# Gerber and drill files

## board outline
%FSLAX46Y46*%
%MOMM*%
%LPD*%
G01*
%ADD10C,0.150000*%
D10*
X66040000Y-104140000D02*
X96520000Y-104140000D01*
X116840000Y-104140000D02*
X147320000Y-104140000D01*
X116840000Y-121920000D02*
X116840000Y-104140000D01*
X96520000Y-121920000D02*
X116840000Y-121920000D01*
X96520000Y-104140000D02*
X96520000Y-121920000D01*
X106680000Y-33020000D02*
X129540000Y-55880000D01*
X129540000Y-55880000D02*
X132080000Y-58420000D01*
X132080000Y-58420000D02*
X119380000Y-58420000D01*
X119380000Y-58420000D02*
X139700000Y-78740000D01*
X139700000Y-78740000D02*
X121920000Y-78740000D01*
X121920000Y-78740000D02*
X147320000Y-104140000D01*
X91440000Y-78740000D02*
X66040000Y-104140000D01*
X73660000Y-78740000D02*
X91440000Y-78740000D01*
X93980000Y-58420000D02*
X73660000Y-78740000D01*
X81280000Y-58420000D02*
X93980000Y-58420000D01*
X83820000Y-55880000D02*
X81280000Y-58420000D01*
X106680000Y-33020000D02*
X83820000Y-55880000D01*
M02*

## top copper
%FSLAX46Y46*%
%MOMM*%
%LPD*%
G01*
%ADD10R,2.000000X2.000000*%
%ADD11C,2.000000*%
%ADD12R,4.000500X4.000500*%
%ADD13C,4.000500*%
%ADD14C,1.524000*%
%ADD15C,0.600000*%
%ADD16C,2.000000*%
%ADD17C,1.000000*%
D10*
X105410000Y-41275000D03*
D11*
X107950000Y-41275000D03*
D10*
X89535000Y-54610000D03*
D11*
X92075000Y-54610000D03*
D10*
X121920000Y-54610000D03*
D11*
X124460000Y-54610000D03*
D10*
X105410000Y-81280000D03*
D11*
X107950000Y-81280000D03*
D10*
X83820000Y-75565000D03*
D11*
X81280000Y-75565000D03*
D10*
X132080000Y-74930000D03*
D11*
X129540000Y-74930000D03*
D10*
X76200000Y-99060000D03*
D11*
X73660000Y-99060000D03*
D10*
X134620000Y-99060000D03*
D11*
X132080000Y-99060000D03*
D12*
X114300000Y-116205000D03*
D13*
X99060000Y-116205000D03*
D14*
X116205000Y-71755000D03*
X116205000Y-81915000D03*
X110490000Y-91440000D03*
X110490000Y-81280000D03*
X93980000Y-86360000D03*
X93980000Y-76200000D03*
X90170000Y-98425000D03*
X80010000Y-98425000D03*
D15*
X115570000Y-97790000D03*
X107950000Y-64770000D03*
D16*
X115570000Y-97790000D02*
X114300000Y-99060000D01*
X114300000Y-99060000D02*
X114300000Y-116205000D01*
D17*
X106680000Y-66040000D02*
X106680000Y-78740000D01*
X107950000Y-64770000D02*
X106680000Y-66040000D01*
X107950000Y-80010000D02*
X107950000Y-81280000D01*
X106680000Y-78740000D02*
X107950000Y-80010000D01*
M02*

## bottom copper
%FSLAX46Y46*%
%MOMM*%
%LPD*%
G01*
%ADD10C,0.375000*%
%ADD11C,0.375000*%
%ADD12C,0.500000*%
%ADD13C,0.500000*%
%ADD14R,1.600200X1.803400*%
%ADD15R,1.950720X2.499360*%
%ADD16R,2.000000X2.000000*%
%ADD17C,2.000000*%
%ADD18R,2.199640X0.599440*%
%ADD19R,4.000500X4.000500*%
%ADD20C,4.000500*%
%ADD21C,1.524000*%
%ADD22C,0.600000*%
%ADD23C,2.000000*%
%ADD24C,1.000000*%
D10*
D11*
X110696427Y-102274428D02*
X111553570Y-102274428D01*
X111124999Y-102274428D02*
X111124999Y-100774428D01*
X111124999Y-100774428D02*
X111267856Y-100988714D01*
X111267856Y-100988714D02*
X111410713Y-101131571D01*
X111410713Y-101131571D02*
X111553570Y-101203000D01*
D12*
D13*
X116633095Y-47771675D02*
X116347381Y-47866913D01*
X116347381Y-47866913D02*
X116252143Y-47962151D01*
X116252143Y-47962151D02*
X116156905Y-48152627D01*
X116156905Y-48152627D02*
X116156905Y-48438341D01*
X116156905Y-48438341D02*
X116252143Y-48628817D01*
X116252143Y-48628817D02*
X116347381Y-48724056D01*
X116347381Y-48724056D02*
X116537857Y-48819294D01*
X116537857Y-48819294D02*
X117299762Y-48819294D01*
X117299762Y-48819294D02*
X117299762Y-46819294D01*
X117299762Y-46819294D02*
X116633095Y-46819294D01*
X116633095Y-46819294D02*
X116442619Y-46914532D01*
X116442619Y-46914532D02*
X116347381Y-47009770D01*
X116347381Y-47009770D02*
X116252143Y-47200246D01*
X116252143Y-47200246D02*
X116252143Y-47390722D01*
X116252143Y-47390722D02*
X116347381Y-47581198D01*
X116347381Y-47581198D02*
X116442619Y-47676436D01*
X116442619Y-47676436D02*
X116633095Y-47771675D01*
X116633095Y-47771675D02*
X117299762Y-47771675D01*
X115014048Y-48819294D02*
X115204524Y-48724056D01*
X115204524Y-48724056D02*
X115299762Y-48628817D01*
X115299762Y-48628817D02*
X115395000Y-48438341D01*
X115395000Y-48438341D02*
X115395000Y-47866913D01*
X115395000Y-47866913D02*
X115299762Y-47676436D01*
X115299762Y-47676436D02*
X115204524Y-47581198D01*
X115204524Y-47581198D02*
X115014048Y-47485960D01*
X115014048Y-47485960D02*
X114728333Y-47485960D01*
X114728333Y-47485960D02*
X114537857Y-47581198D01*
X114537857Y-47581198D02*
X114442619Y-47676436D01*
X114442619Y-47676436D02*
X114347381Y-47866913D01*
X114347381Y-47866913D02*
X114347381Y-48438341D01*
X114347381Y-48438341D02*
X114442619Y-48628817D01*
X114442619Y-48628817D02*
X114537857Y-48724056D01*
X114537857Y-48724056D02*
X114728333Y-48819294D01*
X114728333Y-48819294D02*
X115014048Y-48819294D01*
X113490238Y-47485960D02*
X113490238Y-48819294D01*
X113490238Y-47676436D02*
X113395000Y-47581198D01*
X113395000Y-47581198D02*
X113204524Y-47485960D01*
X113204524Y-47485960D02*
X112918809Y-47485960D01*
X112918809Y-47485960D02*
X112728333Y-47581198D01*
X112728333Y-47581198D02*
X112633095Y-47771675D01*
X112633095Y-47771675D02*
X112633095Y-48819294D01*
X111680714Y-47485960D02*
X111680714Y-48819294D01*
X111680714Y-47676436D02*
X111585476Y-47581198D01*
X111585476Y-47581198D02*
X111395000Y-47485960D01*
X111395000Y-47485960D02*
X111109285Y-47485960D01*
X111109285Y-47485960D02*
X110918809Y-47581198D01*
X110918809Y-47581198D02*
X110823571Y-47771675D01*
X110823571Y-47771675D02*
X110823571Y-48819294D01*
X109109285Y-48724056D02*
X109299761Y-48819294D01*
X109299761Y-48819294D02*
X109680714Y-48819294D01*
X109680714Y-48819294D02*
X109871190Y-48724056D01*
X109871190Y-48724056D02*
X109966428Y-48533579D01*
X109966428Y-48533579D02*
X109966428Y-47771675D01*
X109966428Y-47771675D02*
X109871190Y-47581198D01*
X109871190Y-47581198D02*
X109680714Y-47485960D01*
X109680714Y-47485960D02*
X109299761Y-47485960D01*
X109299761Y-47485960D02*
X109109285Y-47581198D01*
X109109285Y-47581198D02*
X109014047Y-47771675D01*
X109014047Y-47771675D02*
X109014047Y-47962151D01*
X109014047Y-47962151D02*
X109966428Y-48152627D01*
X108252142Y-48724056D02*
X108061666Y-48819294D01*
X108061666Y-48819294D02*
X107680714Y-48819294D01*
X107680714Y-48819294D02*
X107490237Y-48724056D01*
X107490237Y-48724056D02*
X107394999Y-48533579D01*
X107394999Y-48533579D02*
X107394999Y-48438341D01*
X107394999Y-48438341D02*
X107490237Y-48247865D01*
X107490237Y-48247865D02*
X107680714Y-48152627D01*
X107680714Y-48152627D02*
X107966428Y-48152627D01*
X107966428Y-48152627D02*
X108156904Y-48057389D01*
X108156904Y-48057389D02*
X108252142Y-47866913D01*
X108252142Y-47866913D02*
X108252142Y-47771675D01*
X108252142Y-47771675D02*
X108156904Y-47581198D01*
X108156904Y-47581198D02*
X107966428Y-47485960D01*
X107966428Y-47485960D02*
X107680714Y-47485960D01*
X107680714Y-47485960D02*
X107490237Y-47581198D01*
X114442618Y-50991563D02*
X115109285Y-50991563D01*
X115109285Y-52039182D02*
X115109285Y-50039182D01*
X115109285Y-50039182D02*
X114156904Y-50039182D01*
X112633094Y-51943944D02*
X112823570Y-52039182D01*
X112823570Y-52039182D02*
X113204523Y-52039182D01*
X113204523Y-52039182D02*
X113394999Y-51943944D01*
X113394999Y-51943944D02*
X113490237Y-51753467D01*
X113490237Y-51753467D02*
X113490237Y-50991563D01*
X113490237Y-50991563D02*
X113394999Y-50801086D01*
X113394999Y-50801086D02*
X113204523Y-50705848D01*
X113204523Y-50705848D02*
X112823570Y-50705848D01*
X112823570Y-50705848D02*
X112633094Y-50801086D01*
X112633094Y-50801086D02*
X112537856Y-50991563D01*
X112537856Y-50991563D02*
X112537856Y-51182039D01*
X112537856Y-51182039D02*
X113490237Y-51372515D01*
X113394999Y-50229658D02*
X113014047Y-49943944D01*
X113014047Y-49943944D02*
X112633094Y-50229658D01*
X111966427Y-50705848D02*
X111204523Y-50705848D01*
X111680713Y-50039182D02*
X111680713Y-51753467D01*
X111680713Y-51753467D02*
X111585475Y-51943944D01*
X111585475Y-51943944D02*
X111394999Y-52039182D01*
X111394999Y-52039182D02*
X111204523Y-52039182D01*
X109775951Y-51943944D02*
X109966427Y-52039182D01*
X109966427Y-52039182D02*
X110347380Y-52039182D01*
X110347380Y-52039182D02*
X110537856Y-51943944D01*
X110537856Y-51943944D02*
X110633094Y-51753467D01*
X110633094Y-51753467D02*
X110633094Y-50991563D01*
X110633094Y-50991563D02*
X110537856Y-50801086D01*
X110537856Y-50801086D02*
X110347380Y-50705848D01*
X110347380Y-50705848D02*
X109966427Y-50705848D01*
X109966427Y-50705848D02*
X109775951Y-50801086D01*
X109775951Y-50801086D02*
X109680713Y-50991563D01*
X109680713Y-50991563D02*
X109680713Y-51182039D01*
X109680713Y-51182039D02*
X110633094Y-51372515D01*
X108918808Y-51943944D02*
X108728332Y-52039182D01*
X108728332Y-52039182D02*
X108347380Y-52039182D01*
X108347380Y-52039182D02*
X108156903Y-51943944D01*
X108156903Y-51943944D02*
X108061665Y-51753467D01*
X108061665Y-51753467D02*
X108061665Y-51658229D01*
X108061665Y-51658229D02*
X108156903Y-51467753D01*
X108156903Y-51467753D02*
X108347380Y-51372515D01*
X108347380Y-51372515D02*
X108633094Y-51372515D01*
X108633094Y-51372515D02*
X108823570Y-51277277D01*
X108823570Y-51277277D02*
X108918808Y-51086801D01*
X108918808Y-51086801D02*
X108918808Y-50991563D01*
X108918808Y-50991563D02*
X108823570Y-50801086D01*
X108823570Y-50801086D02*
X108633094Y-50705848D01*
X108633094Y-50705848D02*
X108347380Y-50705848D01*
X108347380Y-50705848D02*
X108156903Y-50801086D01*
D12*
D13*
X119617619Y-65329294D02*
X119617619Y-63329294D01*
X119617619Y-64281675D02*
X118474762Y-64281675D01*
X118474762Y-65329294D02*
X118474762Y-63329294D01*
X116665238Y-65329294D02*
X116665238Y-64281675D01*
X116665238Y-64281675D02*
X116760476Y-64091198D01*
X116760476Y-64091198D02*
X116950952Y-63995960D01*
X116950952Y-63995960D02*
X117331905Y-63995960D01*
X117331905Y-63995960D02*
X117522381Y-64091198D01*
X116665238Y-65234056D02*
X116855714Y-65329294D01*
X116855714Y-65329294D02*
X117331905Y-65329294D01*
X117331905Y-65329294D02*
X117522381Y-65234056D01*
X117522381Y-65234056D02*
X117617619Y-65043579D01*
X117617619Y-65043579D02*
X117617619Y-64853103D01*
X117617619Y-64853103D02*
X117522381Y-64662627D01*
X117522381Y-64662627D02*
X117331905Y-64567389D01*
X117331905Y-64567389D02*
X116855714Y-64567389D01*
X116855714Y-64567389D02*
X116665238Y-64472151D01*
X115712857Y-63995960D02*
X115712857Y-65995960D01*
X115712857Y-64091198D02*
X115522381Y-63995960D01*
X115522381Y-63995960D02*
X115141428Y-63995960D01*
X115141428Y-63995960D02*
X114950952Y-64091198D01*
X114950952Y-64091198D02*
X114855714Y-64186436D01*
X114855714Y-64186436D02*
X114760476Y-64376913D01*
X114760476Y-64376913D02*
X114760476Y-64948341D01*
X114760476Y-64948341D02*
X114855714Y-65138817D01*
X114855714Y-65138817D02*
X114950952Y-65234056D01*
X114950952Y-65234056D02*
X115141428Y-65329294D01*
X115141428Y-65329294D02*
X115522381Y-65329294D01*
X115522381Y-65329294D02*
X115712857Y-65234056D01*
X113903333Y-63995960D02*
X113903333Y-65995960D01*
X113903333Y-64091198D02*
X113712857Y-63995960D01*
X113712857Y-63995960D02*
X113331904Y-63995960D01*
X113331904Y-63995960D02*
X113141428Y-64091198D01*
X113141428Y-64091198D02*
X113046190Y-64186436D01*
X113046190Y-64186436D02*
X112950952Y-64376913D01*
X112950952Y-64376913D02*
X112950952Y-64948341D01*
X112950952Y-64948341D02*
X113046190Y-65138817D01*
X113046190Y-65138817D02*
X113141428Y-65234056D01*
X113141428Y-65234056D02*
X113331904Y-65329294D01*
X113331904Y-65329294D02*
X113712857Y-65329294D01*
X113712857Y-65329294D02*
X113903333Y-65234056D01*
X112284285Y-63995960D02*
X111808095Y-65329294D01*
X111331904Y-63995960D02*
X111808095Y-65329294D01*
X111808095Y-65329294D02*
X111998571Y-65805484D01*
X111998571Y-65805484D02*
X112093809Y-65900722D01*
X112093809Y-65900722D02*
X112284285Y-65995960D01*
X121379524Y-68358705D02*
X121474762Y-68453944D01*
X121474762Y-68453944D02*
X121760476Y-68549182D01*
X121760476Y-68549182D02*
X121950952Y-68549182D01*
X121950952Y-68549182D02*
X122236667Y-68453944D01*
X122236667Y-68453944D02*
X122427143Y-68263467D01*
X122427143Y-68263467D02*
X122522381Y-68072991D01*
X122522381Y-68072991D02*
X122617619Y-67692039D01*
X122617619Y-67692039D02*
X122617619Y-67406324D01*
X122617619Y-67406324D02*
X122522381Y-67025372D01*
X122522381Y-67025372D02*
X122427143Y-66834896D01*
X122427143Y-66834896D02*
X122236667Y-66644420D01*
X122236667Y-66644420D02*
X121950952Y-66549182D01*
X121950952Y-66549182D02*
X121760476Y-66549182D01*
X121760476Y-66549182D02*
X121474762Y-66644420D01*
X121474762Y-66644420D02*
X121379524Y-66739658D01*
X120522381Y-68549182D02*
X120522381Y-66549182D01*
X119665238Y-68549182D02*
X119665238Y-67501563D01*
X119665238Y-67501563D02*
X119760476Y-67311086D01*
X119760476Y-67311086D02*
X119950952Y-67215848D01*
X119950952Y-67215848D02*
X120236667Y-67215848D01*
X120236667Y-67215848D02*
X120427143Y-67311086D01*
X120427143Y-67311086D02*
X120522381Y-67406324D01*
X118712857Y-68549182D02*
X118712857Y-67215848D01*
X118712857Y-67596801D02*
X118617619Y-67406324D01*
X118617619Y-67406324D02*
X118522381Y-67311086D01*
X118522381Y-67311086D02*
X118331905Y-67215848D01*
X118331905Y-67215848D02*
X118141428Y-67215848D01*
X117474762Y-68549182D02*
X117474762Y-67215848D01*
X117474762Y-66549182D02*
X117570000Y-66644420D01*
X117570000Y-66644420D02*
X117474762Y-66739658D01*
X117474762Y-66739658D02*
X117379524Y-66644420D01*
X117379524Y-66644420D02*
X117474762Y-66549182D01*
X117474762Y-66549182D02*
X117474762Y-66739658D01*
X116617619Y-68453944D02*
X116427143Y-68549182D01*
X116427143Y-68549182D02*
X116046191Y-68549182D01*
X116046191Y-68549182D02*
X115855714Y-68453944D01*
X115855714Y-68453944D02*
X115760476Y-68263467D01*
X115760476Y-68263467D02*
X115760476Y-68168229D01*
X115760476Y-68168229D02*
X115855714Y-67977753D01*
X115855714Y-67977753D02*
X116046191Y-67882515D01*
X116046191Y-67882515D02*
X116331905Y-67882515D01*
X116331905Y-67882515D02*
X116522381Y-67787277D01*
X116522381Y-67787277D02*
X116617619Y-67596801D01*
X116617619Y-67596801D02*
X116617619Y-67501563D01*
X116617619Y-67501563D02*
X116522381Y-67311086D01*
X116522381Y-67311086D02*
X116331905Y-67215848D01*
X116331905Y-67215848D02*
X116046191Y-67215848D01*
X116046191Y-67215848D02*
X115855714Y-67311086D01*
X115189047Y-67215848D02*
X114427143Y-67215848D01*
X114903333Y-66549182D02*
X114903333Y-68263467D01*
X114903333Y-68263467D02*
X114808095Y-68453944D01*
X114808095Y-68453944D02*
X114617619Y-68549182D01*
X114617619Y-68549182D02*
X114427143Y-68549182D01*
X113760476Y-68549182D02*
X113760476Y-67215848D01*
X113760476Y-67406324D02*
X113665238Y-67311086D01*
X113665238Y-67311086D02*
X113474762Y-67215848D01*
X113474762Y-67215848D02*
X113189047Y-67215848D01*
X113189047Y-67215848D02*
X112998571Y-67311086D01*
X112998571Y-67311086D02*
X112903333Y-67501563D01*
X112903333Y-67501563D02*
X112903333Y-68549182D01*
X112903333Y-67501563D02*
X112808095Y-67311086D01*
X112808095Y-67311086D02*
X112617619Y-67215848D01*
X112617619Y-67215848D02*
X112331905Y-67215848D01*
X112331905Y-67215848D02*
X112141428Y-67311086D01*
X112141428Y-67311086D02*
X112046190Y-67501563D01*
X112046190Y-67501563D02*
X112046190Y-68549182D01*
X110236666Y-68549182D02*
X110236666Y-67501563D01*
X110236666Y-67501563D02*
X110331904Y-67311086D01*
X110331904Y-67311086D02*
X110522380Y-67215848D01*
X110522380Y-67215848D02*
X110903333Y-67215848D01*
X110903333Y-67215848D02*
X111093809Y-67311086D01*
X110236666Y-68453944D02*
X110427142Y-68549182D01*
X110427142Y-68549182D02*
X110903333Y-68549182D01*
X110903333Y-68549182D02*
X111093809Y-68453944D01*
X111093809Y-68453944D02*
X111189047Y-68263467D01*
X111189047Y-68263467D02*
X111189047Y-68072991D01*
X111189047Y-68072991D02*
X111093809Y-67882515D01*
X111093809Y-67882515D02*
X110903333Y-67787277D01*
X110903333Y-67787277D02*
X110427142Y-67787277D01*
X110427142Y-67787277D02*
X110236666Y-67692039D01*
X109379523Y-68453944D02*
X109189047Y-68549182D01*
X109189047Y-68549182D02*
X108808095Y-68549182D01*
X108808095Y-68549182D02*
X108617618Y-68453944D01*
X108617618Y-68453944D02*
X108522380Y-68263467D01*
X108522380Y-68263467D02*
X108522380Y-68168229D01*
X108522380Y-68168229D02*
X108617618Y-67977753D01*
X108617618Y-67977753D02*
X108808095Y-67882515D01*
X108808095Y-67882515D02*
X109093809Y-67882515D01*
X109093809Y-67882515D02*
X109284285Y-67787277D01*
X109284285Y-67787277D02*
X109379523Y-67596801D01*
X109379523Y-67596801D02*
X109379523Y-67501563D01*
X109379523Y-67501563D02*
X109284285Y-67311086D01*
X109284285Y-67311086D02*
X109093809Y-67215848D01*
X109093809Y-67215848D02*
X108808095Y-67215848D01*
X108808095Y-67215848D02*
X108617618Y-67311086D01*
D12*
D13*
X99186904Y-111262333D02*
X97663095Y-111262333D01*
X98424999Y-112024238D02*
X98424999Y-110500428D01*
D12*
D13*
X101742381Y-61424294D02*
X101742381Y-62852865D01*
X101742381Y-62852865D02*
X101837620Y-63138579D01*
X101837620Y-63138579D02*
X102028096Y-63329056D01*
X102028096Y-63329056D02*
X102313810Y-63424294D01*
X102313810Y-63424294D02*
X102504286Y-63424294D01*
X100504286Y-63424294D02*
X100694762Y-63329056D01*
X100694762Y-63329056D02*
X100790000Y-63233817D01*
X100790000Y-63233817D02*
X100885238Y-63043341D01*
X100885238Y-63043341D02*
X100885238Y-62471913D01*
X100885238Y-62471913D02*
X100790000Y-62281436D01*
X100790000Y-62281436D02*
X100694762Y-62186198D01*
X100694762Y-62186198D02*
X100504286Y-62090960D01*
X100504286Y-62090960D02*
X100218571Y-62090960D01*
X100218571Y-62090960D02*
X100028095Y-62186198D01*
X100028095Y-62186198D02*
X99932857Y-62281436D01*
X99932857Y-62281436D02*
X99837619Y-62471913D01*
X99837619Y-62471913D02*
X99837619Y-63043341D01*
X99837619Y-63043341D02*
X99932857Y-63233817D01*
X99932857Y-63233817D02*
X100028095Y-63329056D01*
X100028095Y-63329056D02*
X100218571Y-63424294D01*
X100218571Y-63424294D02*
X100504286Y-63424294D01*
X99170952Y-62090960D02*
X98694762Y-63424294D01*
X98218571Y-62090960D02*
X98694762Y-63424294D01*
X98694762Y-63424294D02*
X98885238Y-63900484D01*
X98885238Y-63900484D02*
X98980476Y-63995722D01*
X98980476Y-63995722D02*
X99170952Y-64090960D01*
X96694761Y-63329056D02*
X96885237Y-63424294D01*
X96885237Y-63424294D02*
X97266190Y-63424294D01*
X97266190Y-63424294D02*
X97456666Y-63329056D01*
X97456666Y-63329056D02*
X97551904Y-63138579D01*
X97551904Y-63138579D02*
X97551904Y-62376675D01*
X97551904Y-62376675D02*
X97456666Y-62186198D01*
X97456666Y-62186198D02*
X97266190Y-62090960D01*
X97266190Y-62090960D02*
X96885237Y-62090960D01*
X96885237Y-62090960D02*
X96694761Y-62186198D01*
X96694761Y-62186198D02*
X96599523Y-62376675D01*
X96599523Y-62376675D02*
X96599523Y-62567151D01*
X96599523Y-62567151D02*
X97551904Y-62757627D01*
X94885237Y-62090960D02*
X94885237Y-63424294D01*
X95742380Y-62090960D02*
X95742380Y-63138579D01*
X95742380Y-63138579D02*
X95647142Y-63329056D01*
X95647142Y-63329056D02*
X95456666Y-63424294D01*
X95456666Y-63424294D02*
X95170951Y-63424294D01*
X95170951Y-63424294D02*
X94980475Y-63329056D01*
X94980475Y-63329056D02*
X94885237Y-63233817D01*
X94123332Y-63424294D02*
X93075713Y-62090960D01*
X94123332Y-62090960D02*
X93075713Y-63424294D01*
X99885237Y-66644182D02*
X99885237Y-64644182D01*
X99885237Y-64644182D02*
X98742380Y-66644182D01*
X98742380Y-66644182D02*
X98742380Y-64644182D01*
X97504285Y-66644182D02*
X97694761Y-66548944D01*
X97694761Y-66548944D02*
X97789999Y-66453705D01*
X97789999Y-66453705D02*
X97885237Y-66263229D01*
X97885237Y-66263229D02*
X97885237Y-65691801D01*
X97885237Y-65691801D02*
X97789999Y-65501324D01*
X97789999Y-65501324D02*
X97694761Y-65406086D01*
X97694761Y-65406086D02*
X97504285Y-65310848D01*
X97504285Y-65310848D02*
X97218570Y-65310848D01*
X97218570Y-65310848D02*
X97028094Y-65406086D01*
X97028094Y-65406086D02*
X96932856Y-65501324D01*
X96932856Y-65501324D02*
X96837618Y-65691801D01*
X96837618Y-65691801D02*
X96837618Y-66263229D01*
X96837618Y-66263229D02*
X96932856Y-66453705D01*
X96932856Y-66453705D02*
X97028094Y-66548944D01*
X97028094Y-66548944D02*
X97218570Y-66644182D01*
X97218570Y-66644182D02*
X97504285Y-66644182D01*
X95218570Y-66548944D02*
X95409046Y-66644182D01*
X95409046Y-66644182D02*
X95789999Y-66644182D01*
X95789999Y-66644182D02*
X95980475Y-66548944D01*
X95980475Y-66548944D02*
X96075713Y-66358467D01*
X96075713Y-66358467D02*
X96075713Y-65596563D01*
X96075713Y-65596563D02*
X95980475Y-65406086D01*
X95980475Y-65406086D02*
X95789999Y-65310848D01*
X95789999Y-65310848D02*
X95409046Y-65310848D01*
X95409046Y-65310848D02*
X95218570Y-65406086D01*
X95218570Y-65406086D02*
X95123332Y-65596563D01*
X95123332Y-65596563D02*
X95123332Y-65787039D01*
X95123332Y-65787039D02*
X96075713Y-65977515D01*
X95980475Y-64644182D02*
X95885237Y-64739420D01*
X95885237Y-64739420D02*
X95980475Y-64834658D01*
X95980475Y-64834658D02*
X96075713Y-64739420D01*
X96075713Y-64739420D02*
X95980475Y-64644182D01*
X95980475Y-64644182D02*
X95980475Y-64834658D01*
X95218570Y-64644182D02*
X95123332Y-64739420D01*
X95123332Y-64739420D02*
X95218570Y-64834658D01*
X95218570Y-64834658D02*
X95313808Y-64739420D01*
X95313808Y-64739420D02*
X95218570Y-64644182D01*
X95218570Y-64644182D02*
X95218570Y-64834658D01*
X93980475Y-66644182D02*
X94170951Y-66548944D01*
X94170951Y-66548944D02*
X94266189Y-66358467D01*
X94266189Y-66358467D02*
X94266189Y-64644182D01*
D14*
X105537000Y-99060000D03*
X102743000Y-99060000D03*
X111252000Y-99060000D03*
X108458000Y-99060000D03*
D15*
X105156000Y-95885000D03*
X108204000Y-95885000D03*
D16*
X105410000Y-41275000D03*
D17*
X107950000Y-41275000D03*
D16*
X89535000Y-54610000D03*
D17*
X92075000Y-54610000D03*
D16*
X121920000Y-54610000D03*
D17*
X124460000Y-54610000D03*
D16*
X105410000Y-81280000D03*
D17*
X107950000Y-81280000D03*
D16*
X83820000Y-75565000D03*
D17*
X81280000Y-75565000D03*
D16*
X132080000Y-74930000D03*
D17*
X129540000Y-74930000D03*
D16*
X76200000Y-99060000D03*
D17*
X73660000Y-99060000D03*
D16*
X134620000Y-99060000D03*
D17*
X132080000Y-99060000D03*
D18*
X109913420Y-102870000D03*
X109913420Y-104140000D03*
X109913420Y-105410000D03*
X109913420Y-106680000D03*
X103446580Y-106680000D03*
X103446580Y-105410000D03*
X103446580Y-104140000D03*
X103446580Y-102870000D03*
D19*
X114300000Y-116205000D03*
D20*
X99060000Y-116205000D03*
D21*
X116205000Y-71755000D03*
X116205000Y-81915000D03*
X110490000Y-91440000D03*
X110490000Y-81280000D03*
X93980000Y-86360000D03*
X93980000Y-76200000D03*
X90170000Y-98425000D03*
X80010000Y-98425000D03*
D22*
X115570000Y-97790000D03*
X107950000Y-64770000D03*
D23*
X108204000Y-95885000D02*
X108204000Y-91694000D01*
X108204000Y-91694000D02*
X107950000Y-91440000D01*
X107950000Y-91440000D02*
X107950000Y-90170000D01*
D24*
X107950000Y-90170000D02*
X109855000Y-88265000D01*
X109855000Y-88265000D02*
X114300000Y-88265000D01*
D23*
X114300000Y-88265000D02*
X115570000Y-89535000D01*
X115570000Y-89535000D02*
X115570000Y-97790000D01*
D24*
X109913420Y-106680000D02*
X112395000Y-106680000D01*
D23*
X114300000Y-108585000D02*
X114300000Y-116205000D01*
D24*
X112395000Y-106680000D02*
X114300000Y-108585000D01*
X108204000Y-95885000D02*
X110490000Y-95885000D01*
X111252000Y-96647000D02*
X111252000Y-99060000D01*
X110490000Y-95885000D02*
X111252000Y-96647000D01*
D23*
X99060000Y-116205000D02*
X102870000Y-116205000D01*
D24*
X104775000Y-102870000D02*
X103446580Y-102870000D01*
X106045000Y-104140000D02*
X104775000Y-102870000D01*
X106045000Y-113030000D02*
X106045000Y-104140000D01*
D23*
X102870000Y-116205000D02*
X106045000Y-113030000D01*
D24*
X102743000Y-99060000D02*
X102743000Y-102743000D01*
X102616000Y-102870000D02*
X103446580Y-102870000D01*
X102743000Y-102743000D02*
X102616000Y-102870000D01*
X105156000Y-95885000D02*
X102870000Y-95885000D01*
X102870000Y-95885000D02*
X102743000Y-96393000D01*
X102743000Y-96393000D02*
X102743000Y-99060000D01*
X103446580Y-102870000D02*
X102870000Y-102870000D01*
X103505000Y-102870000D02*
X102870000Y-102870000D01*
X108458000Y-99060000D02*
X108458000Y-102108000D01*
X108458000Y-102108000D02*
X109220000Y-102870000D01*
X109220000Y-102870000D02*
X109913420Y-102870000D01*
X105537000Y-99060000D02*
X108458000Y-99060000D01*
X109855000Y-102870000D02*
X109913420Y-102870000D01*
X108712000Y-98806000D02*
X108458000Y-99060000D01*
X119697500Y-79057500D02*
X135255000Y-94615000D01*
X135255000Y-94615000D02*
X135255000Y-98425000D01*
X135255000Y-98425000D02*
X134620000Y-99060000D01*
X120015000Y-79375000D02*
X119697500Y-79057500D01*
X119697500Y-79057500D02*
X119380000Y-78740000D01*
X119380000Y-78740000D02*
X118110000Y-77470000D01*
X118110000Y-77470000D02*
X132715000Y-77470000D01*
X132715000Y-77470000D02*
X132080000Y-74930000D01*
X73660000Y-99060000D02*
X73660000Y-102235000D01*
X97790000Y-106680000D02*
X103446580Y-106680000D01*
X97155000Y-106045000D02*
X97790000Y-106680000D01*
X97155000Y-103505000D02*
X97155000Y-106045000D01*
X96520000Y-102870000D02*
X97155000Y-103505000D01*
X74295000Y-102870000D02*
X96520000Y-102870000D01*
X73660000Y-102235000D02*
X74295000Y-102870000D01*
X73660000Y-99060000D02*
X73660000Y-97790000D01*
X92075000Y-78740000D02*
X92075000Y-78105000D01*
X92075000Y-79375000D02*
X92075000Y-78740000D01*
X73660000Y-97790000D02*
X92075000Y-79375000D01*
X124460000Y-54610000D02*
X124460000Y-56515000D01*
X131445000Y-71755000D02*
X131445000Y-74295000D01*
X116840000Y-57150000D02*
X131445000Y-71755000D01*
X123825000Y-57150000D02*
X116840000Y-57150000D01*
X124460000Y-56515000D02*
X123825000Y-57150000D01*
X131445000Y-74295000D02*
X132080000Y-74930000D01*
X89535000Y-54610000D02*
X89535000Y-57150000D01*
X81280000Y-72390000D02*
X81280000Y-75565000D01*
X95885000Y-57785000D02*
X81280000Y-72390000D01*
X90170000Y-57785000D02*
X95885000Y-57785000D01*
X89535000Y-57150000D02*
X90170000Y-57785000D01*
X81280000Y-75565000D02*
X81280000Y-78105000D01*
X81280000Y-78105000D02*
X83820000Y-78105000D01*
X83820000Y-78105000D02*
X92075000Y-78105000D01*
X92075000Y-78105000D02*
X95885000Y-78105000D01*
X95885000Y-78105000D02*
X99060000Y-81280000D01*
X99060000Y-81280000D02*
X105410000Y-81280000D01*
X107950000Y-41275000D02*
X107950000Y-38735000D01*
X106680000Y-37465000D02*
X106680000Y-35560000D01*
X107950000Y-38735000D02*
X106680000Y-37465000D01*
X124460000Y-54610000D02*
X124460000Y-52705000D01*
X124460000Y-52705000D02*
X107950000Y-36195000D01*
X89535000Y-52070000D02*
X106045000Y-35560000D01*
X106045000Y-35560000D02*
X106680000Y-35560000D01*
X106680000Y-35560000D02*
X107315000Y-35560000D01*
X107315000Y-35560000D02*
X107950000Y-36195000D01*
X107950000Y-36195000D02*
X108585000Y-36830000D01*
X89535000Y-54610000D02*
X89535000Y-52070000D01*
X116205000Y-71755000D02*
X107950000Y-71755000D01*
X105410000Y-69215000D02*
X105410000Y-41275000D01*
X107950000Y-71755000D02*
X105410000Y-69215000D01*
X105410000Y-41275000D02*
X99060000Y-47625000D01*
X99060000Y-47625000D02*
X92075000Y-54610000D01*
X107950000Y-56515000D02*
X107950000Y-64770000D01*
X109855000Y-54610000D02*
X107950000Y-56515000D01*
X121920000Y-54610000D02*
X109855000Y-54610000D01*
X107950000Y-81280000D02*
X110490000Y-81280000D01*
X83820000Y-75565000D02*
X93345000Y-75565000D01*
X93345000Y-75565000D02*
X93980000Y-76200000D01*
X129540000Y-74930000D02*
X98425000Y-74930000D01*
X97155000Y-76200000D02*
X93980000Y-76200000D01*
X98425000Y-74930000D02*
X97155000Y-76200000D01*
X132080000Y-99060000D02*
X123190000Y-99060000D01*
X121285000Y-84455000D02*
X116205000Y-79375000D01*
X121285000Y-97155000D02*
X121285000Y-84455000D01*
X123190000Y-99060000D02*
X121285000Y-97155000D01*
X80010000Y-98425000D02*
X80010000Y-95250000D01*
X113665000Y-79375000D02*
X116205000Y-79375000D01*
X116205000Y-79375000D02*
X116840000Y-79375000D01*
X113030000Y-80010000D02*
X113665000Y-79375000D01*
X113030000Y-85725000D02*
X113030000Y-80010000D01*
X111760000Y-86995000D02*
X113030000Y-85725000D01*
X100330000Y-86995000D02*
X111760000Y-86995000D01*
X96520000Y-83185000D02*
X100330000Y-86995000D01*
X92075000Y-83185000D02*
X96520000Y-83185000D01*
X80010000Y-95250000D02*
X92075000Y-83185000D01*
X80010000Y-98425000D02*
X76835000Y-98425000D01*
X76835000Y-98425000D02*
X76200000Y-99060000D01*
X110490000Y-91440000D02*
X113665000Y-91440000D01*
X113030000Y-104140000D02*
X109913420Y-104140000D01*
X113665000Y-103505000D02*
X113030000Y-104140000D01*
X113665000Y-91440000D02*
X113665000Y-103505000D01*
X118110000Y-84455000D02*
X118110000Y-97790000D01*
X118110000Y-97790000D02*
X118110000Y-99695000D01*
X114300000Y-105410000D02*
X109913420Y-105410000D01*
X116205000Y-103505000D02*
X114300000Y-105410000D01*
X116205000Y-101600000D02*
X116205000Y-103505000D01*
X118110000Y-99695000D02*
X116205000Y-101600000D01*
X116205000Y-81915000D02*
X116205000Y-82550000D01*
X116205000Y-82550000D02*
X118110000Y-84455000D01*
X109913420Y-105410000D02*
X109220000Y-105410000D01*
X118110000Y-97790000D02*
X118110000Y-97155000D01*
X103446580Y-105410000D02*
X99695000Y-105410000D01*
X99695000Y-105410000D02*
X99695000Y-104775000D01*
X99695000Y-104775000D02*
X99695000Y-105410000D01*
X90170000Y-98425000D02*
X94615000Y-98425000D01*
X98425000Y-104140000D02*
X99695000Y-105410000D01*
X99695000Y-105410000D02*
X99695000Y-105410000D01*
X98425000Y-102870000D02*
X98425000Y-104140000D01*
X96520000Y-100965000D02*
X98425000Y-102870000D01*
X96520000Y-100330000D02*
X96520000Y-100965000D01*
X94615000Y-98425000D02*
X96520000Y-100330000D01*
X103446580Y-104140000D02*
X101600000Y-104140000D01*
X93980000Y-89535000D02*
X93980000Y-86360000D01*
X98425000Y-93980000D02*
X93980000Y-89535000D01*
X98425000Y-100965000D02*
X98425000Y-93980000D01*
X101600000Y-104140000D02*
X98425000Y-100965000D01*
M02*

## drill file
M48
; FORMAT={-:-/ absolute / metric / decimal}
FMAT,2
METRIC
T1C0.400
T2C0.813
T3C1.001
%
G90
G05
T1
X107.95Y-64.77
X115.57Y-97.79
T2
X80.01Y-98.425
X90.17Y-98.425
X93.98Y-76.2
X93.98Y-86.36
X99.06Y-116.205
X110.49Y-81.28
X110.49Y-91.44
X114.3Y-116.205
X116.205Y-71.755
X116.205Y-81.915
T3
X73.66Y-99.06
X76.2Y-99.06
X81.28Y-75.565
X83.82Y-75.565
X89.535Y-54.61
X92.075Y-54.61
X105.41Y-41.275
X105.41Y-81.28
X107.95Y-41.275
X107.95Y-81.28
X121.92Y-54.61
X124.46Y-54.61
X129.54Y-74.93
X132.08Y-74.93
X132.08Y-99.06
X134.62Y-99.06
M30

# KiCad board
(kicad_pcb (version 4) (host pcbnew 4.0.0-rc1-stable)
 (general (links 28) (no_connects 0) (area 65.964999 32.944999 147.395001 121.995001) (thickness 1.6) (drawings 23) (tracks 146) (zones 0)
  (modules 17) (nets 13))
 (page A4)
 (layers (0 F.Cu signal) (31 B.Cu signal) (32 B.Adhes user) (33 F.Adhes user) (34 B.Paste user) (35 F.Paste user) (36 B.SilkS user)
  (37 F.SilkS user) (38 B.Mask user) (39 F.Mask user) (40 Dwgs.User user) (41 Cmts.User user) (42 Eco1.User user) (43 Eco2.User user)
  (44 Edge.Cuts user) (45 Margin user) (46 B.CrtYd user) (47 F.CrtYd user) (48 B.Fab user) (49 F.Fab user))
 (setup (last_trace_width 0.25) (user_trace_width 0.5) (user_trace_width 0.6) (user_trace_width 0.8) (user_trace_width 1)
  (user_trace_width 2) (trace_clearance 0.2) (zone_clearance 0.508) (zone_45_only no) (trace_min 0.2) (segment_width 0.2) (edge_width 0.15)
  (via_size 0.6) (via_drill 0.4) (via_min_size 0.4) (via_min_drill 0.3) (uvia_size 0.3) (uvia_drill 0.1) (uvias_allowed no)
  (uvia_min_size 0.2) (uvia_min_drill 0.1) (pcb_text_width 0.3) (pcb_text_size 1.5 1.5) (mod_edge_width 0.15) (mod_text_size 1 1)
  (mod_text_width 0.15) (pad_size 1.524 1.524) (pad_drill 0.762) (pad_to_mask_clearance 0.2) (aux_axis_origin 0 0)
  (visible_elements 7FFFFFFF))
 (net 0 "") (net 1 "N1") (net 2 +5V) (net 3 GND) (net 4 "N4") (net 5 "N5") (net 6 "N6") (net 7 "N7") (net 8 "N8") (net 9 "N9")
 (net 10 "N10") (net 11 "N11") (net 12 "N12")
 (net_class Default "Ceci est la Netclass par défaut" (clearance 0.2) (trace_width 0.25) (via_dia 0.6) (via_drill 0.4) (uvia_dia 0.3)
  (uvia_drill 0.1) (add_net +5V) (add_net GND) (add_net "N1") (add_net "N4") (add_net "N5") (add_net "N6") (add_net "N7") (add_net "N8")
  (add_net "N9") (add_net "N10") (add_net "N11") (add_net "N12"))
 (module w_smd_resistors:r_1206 (layer B.Cu) (at 104.14 99.06)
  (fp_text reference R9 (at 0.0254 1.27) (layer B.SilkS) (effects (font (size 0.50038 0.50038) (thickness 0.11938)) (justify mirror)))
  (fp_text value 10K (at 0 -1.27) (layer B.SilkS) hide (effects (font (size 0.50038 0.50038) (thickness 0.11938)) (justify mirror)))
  (pad 1 smd rect (at 1.397 0) (size 1.6002 1.8034) (layers B.Cu B.Paste B.Mask) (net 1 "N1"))
  (pad 2 smd rect (at -1.397 0) (size 1.6002 1.8034) (layers B.Cu B.Paste B.Mask) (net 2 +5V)))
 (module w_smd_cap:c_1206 (layer B.Cu) (at 109.855 99.06)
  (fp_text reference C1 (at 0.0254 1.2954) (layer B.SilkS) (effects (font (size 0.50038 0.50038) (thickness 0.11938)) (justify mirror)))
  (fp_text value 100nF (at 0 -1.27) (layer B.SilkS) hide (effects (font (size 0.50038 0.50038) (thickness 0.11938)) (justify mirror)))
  (pad 1 smd rect (at 1.397 0) (size 1.6002 1.8034) (layers B.Cu B.Paste B.Mask) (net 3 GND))
  (pad 2 smd rect (at -1.397 0) (size 1.6002 1.8034) (layers B.Cu B.Paste B.Mask) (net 1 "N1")))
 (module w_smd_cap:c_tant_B (layer B.Cu) (at 106.68 95.885 180)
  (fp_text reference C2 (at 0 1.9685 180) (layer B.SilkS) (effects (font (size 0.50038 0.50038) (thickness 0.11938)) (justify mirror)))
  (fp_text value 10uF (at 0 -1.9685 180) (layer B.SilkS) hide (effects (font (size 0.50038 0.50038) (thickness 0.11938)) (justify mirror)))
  (pad 1 smd rect (at 1.524 0 180) (size 1.95072 2.49936) (layers B.Cu B.Paste B.Mask) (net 2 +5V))
  (pad 2 smd rect (at -1.524 0 180) (size 1.95072 2.49936) (layers B.Cu B.Paste B.Mask) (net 3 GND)))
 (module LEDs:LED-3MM (layer F.Cu) (at 105.41 41.275)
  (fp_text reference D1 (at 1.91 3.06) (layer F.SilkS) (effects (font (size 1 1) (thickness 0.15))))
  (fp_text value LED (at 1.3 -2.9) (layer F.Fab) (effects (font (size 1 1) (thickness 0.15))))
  (pad 1 thru_hole rect (at 0 0 90) (size 2 2) (drill 1.00076) (layers *.Cu *.Mask F.SilkS) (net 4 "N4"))
  (pad 2 thru_hole circle (at 2.54 0) (size 2 2) (drill 1.00076) (layers *.Cu *.Mask F.SilkS) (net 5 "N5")))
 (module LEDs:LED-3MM (layer F.Cu) (at 89.535 54.61)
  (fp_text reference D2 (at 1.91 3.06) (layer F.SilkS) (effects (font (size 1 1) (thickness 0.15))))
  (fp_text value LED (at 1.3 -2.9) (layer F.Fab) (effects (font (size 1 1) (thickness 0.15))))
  (pad 1 thru_hole rect (at 0 0 90) (size 2 2) (drill 1.00076) (layers *.Cu *.Mask F.SilkS) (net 5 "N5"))
  (pad 2 thru_hole circle (at 2.54 0) (size 2 2) (drill 1.00076) (layers *.Cu *.Mask F.SilkS) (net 4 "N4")))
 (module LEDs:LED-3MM (layer F.Cu) (at 121.92 54.61)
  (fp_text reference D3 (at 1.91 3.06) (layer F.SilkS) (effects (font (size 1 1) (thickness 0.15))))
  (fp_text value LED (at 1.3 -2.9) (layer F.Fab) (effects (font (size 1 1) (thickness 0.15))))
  (pad 1 thru_hole rect (at 0 0 90) (size 2 2) (drill 1.00076) (layers *.Cu *.Mask F.SilkS) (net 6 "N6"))
  (pad 2 thru_hole circle (at 2.54 0) (size 2 2) (drill 1.00076) (layers *.Cu *.Mask F.SilkS) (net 5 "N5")))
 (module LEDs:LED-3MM (layer F.Cu) (at 105.41 81.28)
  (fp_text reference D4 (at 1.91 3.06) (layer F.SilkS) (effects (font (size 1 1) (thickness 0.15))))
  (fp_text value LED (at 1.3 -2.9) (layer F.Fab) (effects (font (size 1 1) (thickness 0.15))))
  (pad 1 thru_hole rect (at 0 0 90) (size 2 2) (drill 1.00076) (layers *.Cu *.Mask F.SilkS) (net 5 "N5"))
  (pad 2 thru_hole circle (at 2.54 0) (size 2 2) (drill 1.00076) (layers *.Cu *.Mask F.SilkS) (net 6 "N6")))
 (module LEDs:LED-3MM (layer F.Cu) (at 83.82 75.565 180)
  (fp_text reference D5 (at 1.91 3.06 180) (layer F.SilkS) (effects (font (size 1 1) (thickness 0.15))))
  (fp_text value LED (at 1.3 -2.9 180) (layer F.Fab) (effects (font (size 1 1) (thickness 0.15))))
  (pad 1 thru_hole rect (at 0 0 270) (size 2 2) (drill 1.00076) (layers *.Cu *.Mask F.SilkS) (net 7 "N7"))
  (pad 2 thru_hole circle (at 2.54 0 180) (size 2 2) (drill 1.00076) (layers *.Cu *.Mask F.SilkS) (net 5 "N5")))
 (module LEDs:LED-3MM (layer F.Cu) (at 132.08 74.93 180)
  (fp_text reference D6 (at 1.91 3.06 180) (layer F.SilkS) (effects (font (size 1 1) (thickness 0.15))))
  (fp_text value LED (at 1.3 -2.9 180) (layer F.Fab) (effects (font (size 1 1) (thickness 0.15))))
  (pad 1 thru_hole rect (at 0 0 270) (size 2 2) (drill 1.00076) (layers *.Cu *.Mask F.SilkS) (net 5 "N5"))
  (pad 2 thru_hole circle (at 2.54 0 180) (size 2 2) (drill 1.00076) (layers *.Cu *.Mask F.SilkS) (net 7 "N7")))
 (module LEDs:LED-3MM (layer F.Cu) (at 76.2 99.06 180)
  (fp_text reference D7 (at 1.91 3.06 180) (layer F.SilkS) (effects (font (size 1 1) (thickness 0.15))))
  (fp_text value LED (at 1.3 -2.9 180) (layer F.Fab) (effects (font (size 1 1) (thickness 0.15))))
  (pad 1 thru_hole rect (at 0 0 270) (size 2 2) (drill 1.00076) (layers *.Cu *.Mask F.SilkS) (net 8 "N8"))
  (pad 2 thru_hole circle (at 2.54 0 180) (size 2 2) (drill 1.00076) (layers *.Cu *.Mask F.SilkS) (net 5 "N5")))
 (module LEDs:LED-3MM (layer F.Cu) (at 134.62 99.06 180)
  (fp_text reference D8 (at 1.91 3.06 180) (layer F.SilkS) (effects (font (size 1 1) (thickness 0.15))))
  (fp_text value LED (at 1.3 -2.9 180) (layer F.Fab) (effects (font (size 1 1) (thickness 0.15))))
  (pad 1 thru_hole rect (at 0 0 270) (size 2 2) (drill 1.00076) (layers *.Cu *.Mask F.SilkS) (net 5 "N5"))
  (pad 2 thru_hole circle (at 2.54 0 180) (size 2 2) (drill 1.00076) (layers *.Cu *.Mask F.SilkS) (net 8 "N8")))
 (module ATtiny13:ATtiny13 (layer B.Cu) (at 106.045 104.775 270)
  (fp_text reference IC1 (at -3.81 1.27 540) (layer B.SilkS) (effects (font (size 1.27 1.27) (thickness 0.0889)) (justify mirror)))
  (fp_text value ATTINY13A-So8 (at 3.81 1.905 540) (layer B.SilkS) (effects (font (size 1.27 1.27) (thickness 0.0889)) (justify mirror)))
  (pad 1 smd rect (at -1.905 -3.86842 270) (size 0.59944 2.19964) (layers B.Cu B.Paste B.Mask) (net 1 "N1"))
  (pad 2 smd rect (at -0.635 -3.86842 270) (size 0.59944 2.19964) (layers B.Cu B.Paste B.Mask) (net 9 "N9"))
  (pad 3 smd rect (at 0.635 -3.86842 270) (size 0.59944 2.19964) (layers B.Cu B.Paste B.Mask) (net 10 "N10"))
  (pad 4 smd rect (at 1.905 -3.86842 270) (size 0.59944 2.19964) (layers B.Cu B.Paste B.Mask) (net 3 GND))
  (pad 5 smd rect (at 1.905 2.59842 270) (size 0.59944 2.19964) (layers B.Cu B.Paste B.Mask) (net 5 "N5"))
  (pad 6 smd rect (at 0.635 2.59842 270) (size 0.59944 2.19964) (layers B.Cu B.Paste B.Mask) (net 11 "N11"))
  (pad 7 smd rect (at -0.635 2.59842 270) (size 0.59944 2.19964) (layers B.Cu B.Paste B.Mask) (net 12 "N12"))
  (pad 8 smd rect (at -1.905 2.59842 270) (size 0.59944 2.19964) (layers B.Cu B.Paste B.Mask) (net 2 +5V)))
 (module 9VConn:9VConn (layer F.Cu) (at 106.68 116.205)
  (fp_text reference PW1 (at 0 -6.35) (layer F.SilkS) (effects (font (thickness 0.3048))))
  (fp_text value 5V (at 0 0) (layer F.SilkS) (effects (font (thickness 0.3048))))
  (pad 1 thru_hole rect (at 7.62 0) (size 4.0005 4.0005) (drill 0.8128) (layers *.Cu *.Mask F.SilkS) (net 3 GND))
  (pad 2 thru_hole circle (at -7.62 0) (size 4.0005 4.0005) (drill 0.8128) (layers *.Cu *.Mask F.SilkS) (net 2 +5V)))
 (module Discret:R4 (layer B.Cu) (at 116.205 76.835 270)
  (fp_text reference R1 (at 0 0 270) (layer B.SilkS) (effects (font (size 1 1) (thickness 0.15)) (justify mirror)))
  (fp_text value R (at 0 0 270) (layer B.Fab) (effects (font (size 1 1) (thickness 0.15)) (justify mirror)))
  (pad 1 thru_hole circle (at -5.08 0 270) (size 1.524 1.524) (drill 0.8128) (layers *.Cu *.Mask B.SilkS) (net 4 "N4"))
  (pad 2 thru_hole circle (at 5.08 0 270) (size 1.524 1.524) (drill 0.8128) (layers *.Cu *.Mask B.SilkS) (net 10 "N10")))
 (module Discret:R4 (layer B.Cu) (at 110.49 86.36 90)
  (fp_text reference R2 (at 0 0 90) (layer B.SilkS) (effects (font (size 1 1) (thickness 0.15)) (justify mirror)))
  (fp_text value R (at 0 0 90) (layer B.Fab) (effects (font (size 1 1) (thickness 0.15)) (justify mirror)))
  (pad 1 thru_hole circle (at -5.08 0 90) (size 1.524 1.524) (drill 0.8128) (layers *.Cu *.Mask B.SilkS) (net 9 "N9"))
  (pad 2 thru_hole circle (at 5.08 0 90) (size 1.524 1.524) (drill 0.8128) (layers *.Cu *.Mask B.SilkS) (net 6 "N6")))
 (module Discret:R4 (layer B.Cu) (at 93.98 81.28 90)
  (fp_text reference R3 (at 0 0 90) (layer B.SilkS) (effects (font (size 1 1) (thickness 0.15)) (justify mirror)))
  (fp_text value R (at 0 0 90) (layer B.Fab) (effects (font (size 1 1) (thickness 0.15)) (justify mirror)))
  (pad 1 thru_hole circle (at -5.08 0 90) (size 1.524 1.524) (drill 0.8128) (layers *.Cu *.Mask B.SilkS) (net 12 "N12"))
  (pad 2 thru_hole circle (at 5.08 0 90) (size 1.524 1.524) (drill 0.8128) (layers *.Cu *.Mask B.SilkS) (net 7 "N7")))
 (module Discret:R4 (layer B.Cu) (at 85.09 98.425 180)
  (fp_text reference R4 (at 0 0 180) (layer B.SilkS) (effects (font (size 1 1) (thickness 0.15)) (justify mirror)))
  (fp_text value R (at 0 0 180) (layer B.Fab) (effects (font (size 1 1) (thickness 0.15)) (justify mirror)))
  (pad 1 thru_hole circle (at -5.08 0 180) (size 1.524 1.524) (drill 0.8128) (layers *.Cu *.Mask B.SilkS) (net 11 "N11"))
  (pad 2 thru_hole circle (at 5.08 0 180) (size 1.524 1.524) (drill 0.8128) (layers *.Cu *.Mask B.SilkS) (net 8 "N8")))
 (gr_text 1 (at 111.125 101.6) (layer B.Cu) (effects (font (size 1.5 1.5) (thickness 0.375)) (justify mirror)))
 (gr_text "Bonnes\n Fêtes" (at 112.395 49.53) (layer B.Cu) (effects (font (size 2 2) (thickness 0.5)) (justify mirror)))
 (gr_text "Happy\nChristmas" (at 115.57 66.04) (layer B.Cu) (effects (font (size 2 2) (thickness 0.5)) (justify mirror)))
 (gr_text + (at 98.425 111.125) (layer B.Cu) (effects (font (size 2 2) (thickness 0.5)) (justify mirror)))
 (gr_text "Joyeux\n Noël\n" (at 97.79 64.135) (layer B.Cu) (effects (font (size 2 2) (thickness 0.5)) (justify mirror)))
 (gr_line (start 66.04 104.14) (end 96.52 104.14) (angle 90) (layer Edge.Cuts) (width 0.15))
 (gr_line (start 116.84 104.14) (end 147.32 104.14) (angle 90) (layer Edge.Cuts) (width 0.15))
 (gr_line (start 116.84 121.92) (end 116.84 104.14) (angle 90) (layer Edge.Cuts) (width 0.15))
 (gr_line (start 96.52 121.92) (end 116.84 121.92) (angle 90) (layer Edge.Cuts) (width 0.15))
 (gr_line (start 96.52 104.14) (end 96.52 121.92) (angle 90) (layer Edge.Cuts) (width 0.15))
 (gr_line (start 106.68 33.02) (end 129.54 55.88) (angle 90) (layer Edge.Cuts) (width 0.15))
 (gr_line (start 129.54 55.88) (end 132.08 58.42) (angle 90) (layer Edge.Cuts) (width 0.15))
 (gr_line (start 132.08 58.42) (end 119.38 58.42) (angle 90) (layer Edge.Cuts) (width 0.15))
 (gr_line (start 119.38 58.42) (end 139.7 78.74) (angle 90) (layer Edge.Cuts) (width 0.15))
 (gr_line (start 139.7 78.74) (end 121.92 78.74) (angle 90) (layer Edge.Cuts) (width 0.15))
 (gr_line (start 121.92 78.74) (end 147.32 104.14) (angle 90) (layer Edge.Cuts) (width 0.15))
 (gr_line (start 91.44 78.74) (end 66.04 104.14) (angle 90) (layer Edge.Cuts) (width 0.15))
 (gr_line (start 73.66 78.74) (end 91.44 78.74) (angle 90) (layer Edge.Cuts) (width 0.15))
 (gr_line (start 93.98 58.42) (end 73.66 78.74) (angle 90) (layer Edge.Cuts) (width 0.15))
 (gr_line (start 81.28 58.42) (end 93.98 58.42) (angle 90) (layer Edge.Cuts) (width 0.15))
 (gr_line (start 83.82 55.88) (end 81.28 58.42) (angle 90) (layer Edge.Cuts) (width 0.15))
 (gr_line (start 106.68 33.02) (end 83.82 55.88) (angle 90) (layer Edge.Cuts) (width 0.15))
 (segment (start 108.204 95.885) (end 108.204 91.694) (width 2) (layer B.Cu) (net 3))
 (segment (start 108.204 91.694) (end 107.95 91.44) (width 2) (layer B.Cu) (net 3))
 (segment (start 107.95 91.44) (end 107.95 90.17) (width 2) (layer B.Cu) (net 3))
 (segment (start 107.95 90.17) (end 109.855 88.265) (width 1) (layer B.Cu) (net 3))
 (segment (start 109.855 88.265) (end 114.3 88.265) (width 1) (layer B.Cu) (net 3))
 (segment (start 114.3 88.265) (end 115.57 89.535) (width 2) (layer B.Cu) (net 3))
 (segment (start 115.57 89.535) (end 115.57 97.79) (width 2) (layer B.Cu) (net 3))
 (via (at 115.57 97.79) (size 0.6) (drill 0.4) (layers F.Cu B.Cu) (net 3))
 (segment (start 115.57 97.79) (end 114.3 99.06) (width 2) (layer F.Cu) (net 3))
 (segment (start 114.3 99.06) (end 114.3 116.205) (width 2) (layer F.Cu) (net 3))
 (segment (start 109.91342 106.68) (end 112.395 106.68) (width 1) (layer B.Cu) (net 3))
 (segment (start 114.3 108.585) (end 114.3 116.205) (width 2) (layer B.Cu) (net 3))
 (segment (start 112.395 106.68) (end 114.3 108.585) (width 1) (layer B.Cu) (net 3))
 (segment (start 108.204 95.885) (end 110.49 95.885) (width 1) (layer B.Cu) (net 3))
 (segment (start 111.252 96.647) (end 111.252 99.06) (width 1) (layer B.Cu) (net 3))
 (segment (start 110.49 95.885) (end 111.252 96.647) (width 1) (layer B.Cu) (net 3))
 (segment (start 99.06 116.205) (end 102.87 116.205) (width 2) (layer B.Cu) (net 2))
 (segment (start 104.775 102.87) (end 103.44658 102.87) (width 1) (layer B.Cu) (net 2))
 (segment (start 106.045 104.14) (end 104.775 102.87) (width 1) (layer B.Cu) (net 2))
 (segment (start 106.045 113.03) (end 106.045 104.14) (width 1) (layer B.Cu) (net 2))
 (segment (start 102.87 116.205) (end 106.045 113.03) (width 2) (layer B.Cu) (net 2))
 (segment (start 102.743 99.06) (end 102.743 102.743) (width 1) (layer B.Cu) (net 2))
 (segment (start 102.616 102.87) (end 103.44658 102.87) (width 1) (layer B.Cu) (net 2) (status 20))
 (segment (start 102.743 102.743) (end 102.616 102.87) (width 1) (layer B.Cu) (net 2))
 (segment (start 105.156 95.885) (end 102.87 95.885) (width 1) (layer B.Cu) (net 2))
 (segment (start 102.87 95.885) (end 102.743 96.393) (width 1) (layer B.Cu) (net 2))
 (segment (start 102.743 96.393) (end 102.743 99.06) (width 1) (layer B.Cu) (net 2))
 (segment (start 103.44658 102.87) (end 102.87 102.87) (width 1) (layer B.Cu) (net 2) (status 10))
 (segment (start 103.505 102.87) (end 102.87 102.87) (width 1) (layer B.Cu) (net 2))
 (segment (start 108.458 99.06) (end 108.458 102.108) (width 1) (layer B.Cu) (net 1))
 (segment (start 108.458 102.108) (end 109.22 102.87) (width 1) (layer B.Cu) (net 1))
 (segment (start 109.22 102.87) (end 109.91342 102.87) (width 1) (layer B.Cu) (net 1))
 (segment (start 105.537 99.06) (end 108.458 99.06) (width 1) (layer B.Cu) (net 1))
 (segment (start 109.855 102.87) (end 109.91342 102.87) (width 1) (layer B.Cu) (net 1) (status 30))
 (segment (start 108.712 98.806) (end 108.458 99.06) (width 1) (layer B.Cu) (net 1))
 (segment (start 119.6975 79.0575) (end 135.255 94.615) (width 1) (layer B.Cu) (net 5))
 (segment (start 135.255 94.615) (end 135.255 98.425) (width 1) (layer B.Cu) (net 5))
 (segment (start 135.255 98.425) (end 134.62 99.06) (width 1) (layer B.Cu) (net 5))
 (segment (start 120.015 79.375) (end 119.6975 79.0575) (width 1) (layer B.Cu) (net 5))
 (segment (start 119.6975 79.0575) (end 119.38 78.74) (width 1) (layer B.Cu) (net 5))
 (segment (start 119.38 78.74) (end 118.11 77.47) (width 1) (layer B.Cu) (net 5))
 (segment (start 118.11 77.47) (end 132.715 77.47) (width 1) (layer B.Cu) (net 5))
 (segment (start 132.715 77.47) (end 132.08 74.93) (width 1) (layer B.Cu) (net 5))
 (segment (start 73.66 99.06) (end 73.66 102.235) (width 1) (layer B.Cu) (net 5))
 (segment (start 97.79 106.68) (end 103.44658 106.68) (width 1) (layer B.Cu) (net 5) (status 20))
 (segment (start 97.155 106.045) (end 97.79 106.68) (width 1) (layer B.Cu) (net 5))
 (segment (start 97.155 103.505) (end 97.155 106.045) (width 1) (layer B.Cu) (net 5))
 (segment (start 96.52 102.87) (end 97.155 103.505) (width 1) (layer B.Cu) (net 5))
 (segment (start 74.295 102.87) (end 96.52 102.87) (width 1) (layer B.Cu) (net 5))
 (segment (start 73.66 102.235) (end 74.295 102.87) (width 1) (layer B.Cu) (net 5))
 (segment (start 73.66 99.06) (end 73.66 97.79) (width 1) (layer B.Cu) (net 5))
 (segment (start 92.075 78.74) (end 92.075 78.105) (width 1) (layer B.Cu) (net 5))
 (segment (start 92.075 79.375) (end 92.075 78.74) (width 1) (layer B.Cu) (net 5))
 (segment (start 73.66 97.79) (end 92.075 79.375) (width 1) (layer B.Cu) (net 5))
 (segment (start 124.46 54.61) (end 124.46 56.515) (width 1) (layer B.Cu) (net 5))
 (segment (start 131.445 71.755) (end 131.445 74.295) (width 1) (layer B.Cu) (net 5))
 (segment (start 116.84 57.15) (end 131.445 71.755) (width 1) (layer B.Cu) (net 5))
 (segment (start 123.825 57.15) (end 116.84 57.15) (width 1) (layer B.Cu) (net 5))
 (segment (start 124.46 56.515) (end 123.825 57.15) (width 1) (layer B.Cu) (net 5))
 (segment (start 131.445 74.295) (end 132.08 74.93) (width 1) (layer B.Cu) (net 5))
 (segment (start 89.535 54.61) (end 89.535 57.15) (width 1) (layer B.Cu) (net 5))
 (segment (start 81.28 72.39) (end 81.28 75.565) (width 1) (layer B.Cu) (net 5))
 (segment (start 95.885 57.785) (end 81.28 72.39) (width 1) (layer B.Cu) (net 5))
 (segment (start 90.17 57.785) (end 95.885 57.785) (width 1) (layer B.Cu) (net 5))
 (segment (start 89.535 57.15) (end 90.17 57.785) (width 1) (layer B.Cu) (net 5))
 (segment (start 81.28 75.565) (end 81.28 78.105) (width 1) (layer B.Cu) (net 5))
 (segment (start 81.28 78.105) (end 83.82 78.105) (width 1) (layer B.Cu) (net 5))
 (segment (start 83.82 78.105) (end 92.075 78.105) (width 1) (layer B.Cu) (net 5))
 (segment (start 92.075 78.105) (end 95.885 78.105) (width 1) (layer B.Cu) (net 5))
 (segment (start 95.885 78.105) (end 99.06 81.28) (width 1) (layer B.Cu) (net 5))
 (segment (start 99.06 81.28) (end 105.41 81.28) (width 1) (layer B.Cu) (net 5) (status 20))
 (segment (start 107.95 41.275) (end 107.95 38.735) (width 1) (layer B.Cu) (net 5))
 (segment (start 106.68 37.465) (end 106.68 35.56) (width 1) (layer B.Cu) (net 5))
 (segment (start 107.95 38.735) (end 106.68 37.465) (width 1) (layer B.Cu) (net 5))
 (segment (start 124.46 54.61) (end 124.46 52.705) (width 1) (layer B.Cu) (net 5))
 (segment (start 124.46 52.705) (end 107.95 36.195) (width 1) (layer B.Cu) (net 5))
 (segment (start 89.535 52.07) (end 106.045 35.56) (width 1) (layer B.Cu) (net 5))
 (segment (start 106.045 35.56) (end 106.68 35.56) (width 1) (layer B.Cu) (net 5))
 (segment (start 106.68 35.56) (end 107.315 35.56) (width 1) (layer B.Cu) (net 5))
 (segment (start 107.315 35.56) (end 107.95 36.195) (width 1) (layer B.Cu) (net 5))
 (segment (start 107.95 36.195) (end 108.585 36.83) (width 1) (layer B.Cu) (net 5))
 (segment (start 89.535 54.61) (end 89.535 52.07) (width 1) (layer B.Cu) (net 5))
 (segment (start 116.205 71.755) (end 107.95 71.755) (width 1) (layer B.Cu) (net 4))
 (segment (start 105.41 69.215) (end 105.41 41.275) (width 1) (layer B.Cu) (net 4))
 (segment (start 107.95 71.755) (end 105.41 69.215) (width 1) (layer B.Cu) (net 4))
 (segment (start 105.41 41.275) (end 99.06 47.625) (width 1) (layer B.Cu) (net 4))
 (segment (start 99.06 47.625) (end 92.075 54.61) (width 1) (layer B.Cu) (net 4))
 (segment (start 106.68 66.04) (end 106.68 78.74) (width 1) (layer F.Cu) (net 6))
 (segment (start 107.95 64.77) (end 106.68 66.04) (width 1) (layer F.Cu) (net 6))
 (via (at 107.95 64.77) (size 0.6) (drill 0.4) (layers F.Cu B.Cu) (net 6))
 (segment (start 107.95 56.515) (end 107.95 64.77) (width 1) (layer B.Cu) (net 6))
 (segment (start 109.855 54.61) (end 107.95 56.515) (width 1) (layer B.Cu) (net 6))
 (segment (start 121.92 54.61) (end 109.855 54.61) (width 1) (layer B.Cu) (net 6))
 (segment (start 107.95 80.01) (end 107.95 81.28) (width 1) (layer F.Cu) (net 6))
 (segment (start 106.68 78.74) (end 107.95 80.01) (width 1) (layer F.Cu) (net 6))
 (segment (start 107.95 81.28) (end 110.49 81.28) (width 1) (layer B.Cu) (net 6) (status 10))
 (segment (start 83.82 75.565) (end 93.345 75.565) (width 1) (layer B.Cu) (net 7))
 (segment (start 93.345 75.565) (end 93.98 76.2) (width 1) (layer B.Cu) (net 7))
 (segment (start 129.54 74.93) (end 98.425 74.93) (width 1) (layer B.Cu) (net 7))
 (segment (start 97.155 76.2) (end 93.98 76.2) (width 1) (layer B.Cu) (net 7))
 (segment (start 98.425 74.93) (end 97.155 76.2) (width 1) (layer B.Cu) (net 7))
 (segment (start 132.08 99.06) (end 123.19 99.06) (width 1) (layer B.Cu) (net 8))
 (segment (start 121.285 84.455) (end 116.205 79.375) (width 1) (layer B.Cu) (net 8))
 (segment (start 121.285 97.155) (end 121.285 84.455) (width 1) (layer B.Cu) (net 8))
 (segment (start 123.19 99.06) (end 121.285 97.155) (width 1) (layer B.Cu) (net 8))
 (segment (start 80.01 98.425) (end 80.01 95.25) (width 1) (layer B.Cu) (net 8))
 (segment (start 113.665 79.375) (end 116.205 79.375) (width 1) (layer B.Cu) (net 8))
 (segment (start 116.205 79.375) (end 116.84 79.375) (width 1) (layer B.Cu) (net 8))
 (segment (start 113.03 80.01) (end 113.665 79.375) (width 1) (layer B.Cu) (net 8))
 (segment (start 113.03 85.725) (end 113.03 80.01) (width 1) (layer B.Cu) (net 8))
 (segment (start 111.76 86.995) (end 113.03 85.725) (width 1) (layer B.Cu) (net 8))
 (segment (start 100.33 86.995) (end 111.76 86.995) (width 1) (layer B.Cu) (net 8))
 (segment (start 96.52 83.185) (end 100.33 86.995) (width 1) (layer B.Cu) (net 8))
 (segment (start 92.075 83.185) (end 96.52 83.185) (width 1) (layer B.Cu) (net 8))
 (segment (start 80.01 95.25) (end 92.075 83.185) (width 1) (layer B.Cu) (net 8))
 (segment (start 80.01 98.425) (end 76.835 98.425) (width 1) (layer B.Cu) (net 8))
 (segment (start 76.835 98.425) (end 76.2 99.06) (width 1) (layer B.Cu) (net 8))
 (segment (start 110.49 91.44) (end 113.665 91.44) (width 1) (layer B.Cu) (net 9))
 (segment (start 113.03 104.14) (end 109.91342 104.14) (width 1) (layer B.Cu) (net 9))
 (segment (start 113.665 103.505) (end 113.03 104.14) (width 1) (layer B.Cu) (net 9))
 (segment (start 113.665 91.44) (end 113.665 103.505) (width 1) (layer B.Cu) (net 9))
 (segment (start 118.11 84.455) (end 118.11 97.79) (width 1) (layer B.Cu) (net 10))
 (segment (start 118.11 97.79) (end 118.11 99.695) (width 1) (layer B.Cu) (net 10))
 (segment (start 114.3 105.41) (end 109.91342 105.41) (width 1) (layer B.Cu) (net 10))
 (segment (start 116.205 103.505) (end 114.3 105.41) (width 1) (layer B.Cu) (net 10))
 (segment (start 116.205 101.6) (end 116.205 103.505) (width 1) (layer B.Cu) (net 10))
 (segment (start 118.11 99.695) (end 116.205 101.6) (width 1) (layer B.Cu) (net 10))
 (segment (start 116.205 81.915) (end 116.205 82.55) (width 1) (layer B.Cu) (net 10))
 (segment (start 116.205 82.55) (end 118.11 84.455) (width 1) (layer B.Cu) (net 10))
 (segment (start 109.91342 105.41) (end 109.22 105.41) (width 1) (layer B.Cu) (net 10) (status 10))
 (segment (start 118.11 97.79) (end 118.11 97.155) (width 1) (layer B.Cu) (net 10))
 (segment (start 103.44658 105.41) (end 99.695 105.41) (width 1) (layer B.Cu) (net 11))
 (segment (start 99.695 105.41) (end 99.695 104.775) (width 1) (layer B.Cu) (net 11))
 (segment (start 99.695 104.775) (end 99.695 105.41) (width 1) (layer B.Cu) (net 11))
 (segment (start 90.17 98.425) (end 94.615 98.425) (width 1) (layer B.Cu) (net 11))
 (segment (start 98.425 104.14) (end 99.695 105.41) (width 1) (layer B.Cu) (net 11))
 (segment (start 99.695 105.41) (end 99.695 105.41) (width 1) (layer B.Cu) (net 11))
 (segment (start 98.425 102.87) (end 98.425 104.14) (width 1) (layer B.Cu) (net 11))
 (segment (start 96.52 100.965) (end 98.425 102.87) (width 1) (layer B.Cu) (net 11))
 (segment (start 96.52 100.33) (end 96.52 100.965) (width 1) (layer B.Cu) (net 11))
 (segment (start 94.615 98.425) (end 96.52 100.33) (width 1) (layer B.Cu) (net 11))
 (segment (start 103.44658 104.14) (end 101.6 104.14) (width 1) (layer B.Cu) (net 12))
 (segment (start 93.98 89.535) (end 93.98 86.36) (width 1) (layer B.Cu) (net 12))
 (segment (start 98.425 93.98) (end 93.98 89.535) (width 1) (layer B.Cu) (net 12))
 (segment (start 98.425 100.965) (end 98.425 93.98) (width 1) (layer B.Cu) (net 12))
 (segment (start 101.6 104.14) (end 98.425 100.965) (width 1) (layer B.Cu) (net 12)))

